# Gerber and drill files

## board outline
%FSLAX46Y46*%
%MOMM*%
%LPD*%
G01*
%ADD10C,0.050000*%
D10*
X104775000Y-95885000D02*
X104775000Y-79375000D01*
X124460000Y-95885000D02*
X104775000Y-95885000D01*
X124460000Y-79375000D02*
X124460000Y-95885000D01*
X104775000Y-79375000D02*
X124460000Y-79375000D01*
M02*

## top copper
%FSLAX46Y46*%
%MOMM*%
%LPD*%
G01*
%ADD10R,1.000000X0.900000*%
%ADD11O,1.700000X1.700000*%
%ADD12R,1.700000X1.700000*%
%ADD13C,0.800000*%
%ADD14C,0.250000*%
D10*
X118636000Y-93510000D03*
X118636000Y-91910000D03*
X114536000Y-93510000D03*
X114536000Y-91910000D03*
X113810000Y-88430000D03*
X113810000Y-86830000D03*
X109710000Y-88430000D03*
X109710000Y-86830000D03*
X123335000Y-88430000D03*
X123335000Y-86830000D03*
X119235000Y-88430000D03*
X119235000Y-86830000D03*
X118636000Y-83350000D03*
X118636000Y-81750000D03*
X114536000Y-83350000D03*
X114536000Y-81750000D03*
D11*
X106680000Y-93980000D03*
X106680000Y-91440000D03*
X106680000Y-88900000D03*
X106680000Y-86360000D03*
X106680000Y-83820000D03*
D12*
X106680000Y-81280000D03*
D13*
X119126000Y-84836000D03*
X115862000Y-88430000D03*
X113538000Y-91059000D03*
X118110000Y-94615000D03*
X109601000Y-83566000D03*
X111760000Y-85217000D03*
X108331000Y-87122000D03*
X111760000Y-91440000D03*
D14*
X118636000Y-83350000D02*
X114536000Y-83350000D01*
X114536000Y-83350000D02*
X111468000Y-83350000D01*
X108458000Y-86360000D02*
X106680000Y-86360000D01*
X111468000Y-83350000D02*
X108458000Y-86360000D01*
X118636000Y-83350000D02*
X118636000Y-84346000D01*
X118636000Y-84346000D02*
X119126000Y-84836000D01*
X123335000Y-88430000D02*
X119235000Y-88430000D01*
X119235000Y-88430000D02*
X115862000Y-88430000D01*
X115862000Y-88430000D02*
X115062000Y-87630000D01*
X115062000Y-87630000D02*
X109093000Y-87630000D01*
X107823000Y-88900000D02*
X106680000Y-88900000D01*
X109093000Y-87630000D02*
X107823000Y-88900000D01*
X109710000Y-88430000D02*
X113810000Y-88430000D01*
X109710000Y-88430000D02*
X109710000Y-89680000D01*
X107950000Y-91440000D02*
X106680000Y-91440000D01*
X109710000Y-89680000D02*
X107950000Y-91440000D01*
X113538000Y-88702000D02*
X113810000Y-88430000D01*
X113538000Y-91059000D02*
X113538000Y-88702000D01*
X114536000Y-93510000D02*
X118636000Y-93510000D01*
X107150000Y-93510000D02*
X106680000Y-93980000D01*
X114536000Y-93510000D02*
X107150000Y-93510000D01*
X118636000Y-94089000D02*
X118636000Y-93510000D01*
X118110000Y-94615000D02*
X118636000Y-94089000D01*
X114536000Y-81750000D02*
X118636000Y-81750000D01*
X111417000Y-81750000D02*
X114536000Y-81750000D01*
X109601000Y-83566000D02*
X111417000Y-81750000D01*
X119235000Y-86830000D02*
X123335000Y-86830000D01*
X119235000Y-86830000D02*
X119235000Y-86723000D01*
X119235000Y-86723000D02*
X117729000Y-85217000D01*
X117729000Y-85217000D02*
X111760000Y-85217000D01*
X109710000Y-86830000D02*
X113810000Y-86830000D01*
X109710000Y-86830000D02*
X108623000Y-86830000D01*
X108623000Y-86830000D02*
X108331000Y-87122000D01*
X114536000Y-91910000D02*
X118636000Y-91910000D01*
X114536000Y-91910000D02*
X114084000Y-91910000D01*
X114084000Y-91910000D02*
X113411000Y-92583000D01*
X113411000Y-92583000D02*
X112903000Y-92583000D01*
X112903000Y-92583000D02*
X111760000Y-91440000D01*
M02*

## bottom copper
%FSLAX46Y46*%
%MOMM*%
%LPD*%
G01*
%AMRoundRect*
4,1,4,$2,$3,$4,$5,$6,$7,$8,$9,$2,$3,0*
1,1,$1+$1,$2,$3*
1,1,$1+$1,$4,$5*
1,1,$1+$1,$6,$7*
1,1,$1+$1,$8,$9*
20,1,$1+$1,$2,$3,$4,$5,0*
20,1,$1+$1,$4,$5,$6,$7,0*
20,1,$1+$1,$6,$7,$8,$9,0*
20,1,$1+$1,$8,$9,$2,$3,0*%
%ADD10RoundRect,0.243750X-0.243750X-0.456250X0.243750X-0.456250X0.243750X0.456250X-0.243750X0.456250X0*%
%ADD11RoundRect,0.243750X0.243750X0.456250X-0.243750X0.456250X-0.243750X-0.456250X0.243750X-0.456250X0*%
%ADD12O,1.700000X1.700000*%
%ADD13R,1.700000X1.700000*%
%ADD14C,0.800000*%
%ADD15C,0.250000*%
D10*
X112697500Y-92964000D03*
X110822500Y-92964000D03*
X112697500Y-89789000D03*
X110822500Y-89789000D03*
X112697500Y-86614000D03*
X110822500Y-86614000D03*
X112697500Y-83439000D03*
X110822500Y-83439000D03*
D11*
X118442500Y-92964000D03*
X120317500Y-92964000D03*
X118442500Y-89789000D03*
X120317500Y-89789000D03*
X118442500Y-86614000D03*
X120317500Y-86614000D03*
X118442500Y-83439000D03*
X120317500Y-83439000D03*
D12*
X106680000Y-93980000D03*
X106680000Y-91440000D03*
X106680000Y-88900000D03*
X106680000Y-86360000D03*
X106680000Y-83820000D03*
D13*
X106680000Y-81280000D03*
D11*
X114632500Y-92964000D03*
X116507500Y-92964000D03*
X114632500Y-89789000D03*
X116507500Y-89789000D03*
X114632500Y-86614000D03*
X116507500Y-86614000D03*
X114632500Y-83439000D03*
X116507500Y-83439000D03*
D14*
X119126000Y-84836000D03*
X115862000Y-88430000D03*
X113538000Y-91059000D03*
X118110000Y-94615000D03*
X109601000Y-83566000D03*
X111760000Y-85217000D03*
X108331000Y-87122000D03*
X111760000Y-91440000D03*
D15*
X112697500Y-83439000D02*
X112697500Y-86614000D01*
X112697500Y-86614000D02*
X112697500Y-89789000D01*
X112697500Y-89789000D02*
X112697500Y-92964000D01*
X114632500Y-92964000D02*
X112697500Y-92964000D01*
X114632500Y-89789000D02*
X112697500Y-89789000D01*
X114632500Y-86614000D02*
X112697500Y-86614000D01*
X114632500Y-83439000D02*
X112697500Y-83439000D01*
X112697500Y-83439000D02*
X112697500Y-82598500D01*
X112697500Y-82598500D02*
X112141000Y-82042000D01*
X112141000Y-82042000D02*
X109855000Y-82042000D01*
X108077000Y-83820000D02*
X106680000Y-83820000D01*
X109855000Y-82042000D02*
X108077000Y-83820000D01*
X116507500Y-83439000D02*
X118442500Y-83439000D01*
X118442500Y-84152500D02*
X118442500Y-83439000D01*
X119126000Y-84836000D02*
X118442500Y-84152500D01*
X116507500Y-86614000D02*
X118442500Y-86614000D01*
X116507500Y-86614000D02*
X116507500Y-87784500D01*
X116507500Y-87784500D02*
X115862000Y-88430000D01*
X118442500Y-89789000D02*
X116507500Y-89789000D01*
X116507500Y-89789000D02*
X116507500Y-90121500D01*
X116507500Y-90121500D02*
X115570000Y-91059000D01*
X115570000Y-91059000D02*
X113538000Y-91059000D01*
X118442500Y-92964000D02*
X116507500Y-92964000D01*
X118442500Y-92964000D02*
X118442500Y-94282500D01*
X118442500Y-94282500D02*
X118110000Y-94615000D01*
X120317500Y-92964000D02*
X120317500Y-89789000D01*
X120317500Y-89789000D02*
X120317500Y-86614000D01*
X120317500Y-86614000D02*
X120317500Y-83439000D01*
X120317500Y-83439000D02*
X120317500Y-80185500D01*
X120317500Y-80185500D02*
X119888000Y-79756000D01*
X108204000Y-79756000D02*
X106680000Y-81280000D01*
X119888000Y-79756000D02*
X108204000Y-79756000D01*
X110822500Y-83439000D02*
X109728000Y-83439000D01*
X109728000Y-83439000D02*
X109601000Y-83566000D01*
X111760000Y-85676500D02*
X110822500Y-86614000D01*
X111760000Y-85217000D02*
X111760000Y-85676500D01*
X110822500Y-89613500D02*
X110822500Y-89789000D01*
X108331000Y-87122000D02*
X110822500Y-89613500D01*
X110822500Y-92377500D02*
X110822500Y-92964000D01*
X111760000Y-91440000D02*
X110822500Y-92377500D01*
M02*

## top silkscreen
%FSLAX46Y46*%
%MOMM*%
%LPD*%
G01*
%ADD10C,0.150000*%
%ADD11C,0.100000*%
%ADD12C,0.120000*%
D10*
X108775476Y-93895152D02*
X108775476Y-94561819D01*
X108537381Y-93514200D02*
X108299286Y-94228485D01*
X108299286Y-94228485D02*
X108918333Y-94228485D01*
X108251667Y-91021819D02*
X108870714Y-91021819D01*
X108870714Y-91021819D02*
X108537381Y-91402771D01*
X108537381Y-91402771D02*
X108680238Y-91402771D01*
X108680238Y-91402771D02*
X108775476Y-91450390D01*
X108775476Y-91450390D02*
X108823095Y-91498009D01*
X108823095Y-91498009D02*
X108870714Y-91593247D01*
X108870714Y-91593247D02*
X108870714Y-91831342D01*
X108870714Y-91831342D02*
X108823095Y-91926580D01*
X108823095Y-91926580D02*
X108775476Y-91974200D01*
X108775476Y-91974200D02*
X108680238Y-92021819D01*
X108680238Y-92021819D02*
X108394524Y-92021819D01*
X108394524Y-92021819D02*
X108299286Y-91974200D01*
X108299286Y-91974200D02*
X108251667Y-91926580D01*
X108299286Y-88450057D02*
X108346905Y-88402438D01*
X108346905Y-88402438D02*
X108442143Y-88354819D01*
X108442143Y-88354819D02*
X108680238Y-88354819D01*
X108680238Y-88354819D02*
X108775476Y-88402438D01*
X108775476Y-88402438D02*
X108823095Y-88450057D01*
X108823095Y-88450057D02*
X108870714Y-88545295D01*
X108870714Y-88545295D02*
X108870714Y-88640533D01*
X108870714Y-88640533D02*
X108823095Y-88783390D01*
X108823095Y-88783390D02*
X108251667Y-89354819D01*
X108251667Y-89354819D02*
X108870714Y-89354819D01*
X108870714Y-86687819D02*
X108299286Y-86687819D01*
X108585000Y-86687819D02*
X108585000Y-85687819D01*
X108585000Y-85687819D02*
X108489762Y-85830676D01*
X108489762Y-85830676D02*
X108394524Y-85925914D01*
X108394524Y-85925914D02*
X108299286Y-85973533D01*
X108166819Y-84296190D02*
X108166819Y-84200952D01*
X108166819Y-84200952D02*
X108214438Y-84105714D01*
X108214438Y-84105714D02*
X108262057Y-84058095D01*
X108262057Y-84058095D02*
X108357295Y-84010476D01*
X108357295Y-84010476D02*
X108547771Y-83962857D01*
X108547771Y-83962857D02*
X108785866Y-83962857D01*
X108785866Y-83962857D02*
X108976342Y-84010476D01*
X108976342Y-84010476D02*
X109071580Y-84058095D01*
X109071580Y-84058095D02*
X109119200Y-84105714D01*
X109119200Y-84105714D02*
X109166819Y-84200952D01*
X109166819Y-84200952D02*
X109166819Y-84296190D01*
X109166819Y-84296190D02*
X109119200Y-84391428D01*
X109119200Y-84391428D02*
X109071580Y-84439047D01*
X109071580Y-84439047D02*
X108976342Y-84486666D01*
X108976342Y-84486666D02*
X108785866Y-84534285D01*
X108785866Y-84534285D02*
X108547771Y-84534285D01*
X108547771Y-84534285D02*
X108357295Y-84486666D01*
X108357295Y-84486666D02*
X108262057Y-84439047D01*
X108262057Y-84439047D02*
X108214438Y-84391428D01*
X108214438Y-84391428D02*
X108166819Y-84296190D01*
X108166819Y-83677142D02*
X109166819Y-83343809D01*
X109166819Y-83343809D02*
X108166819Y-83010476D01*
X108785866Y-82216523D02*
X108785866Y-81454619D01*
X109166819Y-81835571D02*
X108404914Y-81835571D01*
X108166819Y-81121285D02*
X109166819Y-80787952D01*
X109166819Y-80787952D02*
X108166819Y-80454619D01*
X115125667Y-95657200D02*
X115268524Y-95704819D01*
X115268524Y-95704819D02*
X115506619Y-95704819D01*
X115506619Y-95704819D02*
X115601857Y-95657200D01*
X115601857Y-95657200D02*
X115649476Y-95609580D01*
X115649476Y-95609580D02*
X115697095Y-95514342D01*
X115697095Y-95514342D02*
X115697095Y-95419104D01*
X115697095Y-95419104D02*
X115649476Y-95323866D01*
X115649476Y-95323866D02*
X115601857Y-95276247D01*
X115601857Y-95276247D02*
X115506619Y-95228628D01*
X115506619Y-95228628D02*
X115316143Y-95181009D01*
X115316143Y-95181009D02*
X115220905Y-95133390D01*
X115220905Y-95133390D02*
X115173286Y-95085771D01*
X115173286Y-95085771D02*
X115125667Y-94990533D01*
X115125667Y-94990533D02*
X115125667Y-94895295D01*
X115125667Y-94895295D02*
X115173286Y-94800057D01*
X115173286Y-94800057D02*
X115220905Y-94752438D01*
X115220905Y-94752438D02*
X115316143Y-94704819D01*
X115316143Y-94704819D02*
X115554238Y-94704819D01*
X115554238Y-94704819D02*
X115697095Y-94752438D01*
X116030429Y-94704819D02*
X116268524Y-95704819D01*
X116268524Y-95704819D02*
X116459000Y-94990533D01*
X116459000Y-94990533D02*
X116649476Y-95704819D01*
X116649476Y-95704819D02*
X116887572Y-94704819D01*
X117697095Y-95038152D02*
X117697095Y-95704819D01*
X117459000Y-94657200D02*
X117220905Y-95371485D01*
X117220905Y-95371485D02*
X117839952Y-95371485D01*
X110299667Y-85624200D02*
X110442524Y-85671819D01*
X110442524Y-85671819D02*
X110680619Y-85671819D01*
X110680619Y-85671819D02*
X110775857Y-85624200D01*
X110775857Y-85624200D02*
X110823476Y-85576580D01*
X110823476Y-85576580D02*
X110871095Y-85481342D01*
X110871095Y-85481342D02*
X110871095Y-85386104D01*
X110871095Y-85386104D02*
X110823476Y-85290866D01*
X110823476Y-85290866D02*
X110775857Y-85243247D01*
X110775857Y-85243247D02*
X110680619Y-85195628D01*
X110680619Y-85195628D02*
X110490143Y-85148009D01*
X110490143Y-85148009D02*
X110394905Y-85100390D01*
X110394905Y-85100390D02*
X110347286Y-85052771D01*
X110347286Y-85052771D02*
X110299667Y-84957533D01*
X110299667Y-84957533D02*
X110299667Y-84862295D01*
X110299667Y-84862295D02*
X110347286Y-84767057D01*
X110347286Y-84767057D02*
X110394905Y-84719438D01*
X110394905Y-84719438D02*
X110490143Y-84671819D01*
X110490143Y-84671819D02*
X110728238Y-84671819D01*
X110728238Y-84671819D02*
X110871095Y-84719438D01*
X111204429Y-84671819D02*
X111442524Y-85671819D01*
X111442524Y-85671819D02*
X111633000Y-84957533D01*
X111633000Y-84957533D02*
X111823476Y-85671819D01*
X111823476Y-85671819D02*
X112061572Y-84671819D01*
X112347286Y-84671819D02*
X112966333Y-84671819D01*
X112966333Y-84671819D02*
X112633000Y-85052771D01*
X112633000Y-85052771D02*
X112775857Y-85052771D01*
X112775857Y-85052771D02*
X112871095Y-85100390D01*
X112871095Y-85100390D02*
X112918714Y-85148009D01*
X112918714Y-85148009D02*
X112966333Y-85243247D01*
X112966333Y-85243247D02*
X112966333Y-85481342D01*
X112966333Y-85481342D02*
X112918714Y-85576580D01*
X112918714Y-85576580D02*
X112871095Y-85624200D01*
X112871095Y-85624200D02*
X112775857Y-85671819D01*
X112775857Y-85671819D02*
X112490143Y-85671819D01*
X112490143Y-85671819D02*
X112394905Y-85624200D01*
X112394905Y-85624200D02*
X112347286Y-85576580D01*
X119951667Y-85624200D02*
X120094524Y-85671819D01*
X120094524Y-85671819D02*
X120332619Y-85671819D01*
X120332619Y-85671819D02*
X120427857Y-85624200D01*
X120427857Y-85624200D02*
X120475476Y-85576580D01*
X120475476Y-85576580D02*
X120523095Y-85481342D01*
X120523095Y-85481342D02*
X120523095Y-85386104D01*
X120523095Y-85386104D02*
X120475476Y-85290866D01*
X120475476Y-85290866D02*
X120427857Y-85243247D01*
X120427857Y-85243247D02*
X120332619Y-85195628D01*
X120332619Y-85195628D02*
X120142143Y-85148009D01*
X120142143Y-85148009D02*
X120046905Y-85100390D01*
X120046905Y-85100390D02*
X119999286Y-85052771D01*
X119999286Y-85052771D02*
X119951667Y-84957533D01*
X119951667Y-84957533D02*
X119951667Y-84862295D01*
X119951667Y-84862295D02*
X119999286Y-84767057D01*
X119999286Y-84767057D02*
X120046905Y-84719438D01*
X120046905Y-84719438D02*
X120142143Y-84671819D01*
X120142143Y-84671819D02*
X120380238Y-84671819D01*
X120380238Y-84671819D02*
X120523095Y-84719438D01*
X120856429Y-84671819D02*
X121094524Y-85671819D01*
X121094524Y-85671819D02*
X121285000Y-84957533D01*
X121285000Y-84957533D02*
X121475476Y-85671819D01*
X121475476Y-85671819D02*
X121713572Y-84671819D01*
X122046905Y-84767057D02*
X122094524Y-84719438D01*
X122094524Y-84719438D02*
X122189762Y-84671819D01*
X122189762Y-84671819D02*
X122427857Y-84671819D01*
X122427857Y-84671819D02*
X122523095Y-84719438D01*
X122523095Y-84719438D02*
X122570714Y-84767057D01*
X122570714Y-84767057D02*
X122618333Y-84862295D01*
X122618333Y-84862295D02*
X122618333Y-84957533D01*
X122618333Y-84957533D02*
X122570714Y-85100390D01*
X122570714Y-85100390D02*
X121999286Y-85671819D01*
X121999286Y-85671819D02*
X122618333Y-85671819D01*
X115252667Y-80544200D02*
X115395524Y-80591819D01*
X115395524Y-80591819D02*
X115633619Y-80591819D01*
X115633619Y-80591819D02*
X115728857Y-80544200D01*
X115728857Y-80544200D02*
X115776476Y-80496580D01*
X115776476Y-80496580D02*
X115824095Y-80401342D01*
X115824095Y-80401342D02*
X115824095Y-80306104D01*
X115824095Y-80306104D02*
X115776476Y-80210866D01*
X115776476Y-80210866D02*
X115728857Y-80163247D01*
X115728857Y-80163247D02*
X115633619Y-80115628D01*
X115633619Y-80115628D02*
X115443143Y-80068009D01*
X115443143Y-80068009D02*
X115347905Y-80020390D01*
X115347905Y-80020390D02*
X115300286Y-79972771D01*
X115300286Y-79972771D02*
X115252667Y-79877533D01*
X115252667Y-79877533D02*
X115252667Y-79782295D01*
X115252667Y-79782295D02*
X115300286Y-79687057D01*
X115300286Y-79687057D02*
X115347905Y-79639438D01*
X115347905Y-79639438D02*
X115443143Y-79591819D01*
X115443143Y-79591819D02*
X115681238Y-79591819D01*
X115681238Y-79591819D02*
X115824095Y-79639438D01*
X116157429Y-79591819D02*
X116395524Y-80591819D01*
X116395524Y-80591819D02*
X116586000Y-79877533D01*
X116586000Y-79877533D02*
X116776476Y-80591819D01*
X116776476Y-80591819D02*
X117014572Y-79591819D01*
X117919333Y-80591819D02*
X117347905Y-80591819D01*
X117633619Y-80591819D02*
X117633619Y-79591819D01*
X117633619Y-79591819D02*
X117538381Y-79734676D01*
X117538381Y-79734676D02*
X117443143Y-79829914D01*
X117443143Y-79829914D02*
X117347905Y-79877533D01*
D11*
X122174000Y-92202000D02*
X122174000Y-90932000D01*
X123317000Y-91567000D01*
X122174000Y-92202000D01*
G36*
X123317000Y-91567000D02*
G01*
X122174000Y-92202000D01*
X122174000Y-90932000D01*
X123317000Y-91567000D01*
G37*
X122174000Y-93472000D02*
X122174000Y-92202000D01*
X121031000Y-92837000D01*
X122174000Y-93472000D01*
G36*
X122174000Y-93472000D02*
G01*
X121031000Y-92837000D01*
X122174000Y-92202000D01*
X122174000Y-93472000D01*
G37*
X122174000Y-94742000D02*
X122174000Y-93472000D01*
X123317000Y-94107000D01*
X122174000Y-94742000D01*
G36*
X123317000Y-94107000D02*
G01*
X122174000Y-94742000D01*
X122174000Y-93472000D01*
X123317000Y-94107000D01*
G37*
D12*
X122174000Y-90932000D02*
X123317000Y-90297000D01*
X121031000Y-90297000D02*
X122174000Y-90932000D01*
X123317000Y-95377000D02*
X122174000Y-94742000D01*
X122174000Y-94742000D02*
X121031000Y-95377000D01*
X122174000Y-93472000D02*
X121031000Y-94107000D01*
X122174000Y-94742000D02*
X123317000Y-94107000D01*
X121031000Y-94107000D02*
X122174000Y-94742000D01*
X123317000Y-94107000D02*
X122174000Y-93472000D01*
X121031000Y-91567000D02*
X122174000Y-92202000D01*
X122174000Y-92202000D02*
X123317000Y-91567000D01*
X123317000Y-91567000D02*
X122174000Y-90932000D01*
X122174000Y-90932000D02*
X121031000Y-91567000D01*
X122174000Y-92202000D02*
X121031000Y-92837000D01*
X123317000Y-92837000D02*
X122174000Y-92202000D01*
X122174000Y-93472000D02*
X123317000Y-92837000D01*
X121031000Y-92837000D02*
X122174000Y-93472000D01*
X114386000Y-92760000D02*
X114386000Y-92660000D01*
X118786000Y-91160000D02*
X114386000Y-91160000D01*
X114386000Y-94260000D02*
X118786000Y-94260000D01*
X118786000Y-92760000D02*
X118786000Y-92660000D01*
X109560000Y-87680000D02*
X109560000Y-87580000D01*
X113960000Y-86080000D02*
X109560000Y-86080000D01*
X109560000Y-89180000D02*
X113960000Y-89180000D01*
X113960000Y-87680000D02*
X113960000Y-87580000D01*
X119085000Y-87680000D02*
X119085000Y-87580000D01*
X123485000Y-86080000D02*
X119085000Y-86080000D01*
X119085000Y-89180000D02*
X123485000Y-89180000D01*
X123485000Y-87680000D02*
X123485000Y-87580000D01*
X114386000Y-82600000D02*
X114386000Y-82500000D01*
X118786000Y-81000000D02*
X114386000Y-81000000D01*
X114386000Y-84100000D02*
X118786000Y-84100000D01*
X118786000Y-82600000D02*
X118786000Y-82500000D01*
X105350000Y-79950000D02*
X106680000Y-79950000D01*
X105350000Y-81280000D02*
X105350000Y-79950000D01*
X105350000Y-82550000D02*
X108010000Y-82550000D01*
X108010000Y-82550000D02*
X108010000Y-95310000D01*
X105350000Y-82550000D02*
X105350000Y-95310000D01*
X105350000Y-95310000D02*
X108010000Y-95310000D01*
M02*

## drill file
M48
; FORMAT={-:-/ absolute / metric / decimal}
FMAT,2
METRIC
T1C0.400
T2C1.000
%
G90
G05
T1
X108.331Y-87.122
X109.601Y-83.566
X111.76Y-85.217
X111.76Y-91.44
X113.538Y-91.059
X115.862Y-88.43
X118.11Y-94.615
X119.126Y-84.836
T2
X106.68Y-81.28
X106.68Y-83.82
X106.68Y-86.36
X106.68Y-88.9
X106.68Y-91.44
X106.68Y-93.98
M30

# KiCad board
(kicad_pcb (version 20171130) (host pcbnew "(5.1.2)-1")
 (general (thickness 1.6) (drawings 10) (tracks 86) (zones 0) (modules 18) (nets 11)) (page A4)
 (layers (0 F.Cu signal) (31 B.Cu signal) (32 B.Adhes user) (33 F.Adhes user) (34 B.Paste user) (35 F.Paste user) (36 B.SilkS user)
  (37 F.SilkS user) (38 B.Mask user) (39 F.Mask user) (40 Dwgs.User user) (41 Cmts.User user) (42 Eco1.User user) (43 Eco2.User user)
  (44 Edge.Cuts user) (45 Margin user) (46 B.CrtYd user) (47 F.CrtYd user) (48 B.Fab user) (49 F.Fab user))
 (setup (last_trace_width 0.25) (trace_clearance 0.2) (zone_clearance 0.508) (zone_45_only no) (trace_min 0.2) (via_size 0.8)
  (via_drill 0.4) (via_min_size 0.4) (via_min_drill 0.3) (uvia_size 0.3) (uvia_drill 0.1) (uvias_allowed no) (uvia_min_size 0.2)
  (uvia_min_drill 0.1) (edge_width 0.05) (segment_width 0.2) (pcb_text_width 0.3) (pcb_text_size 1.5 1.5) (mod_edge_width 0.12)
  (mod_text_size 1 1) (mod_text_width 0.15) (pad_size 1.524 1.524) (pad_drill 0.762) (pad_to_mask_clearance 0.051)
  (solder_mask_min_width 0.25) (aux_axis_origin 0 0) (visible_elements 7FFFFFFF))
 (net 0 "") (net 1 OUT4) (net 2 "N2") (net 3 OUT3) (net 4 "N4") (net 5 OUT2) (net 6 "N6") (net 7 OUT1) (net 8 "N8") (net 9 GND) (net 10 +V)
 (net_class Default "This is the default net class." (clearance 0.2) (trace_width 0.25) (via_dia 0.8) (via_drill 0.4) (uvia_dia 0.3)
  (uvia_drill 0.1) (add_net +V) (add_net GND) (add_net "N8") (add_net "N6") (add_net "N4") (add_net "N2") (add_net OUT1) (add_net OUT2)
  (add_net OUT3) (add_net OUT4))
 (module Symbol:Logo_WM (layer F.Cu) (at 122.174 92.837 90)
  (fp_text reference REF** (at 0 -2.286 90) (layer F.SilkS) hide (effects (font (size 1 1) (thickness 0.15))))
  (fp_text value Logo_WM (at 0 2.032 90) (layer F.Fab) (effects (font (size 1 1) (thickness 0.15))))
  (fp_poly (pts (xy 0.635 0) (xy 1.905 0) (xy 1.27 1.143)) (layer F.SilkS) (width 0.1))
  (fp_poly (pts (xy -0.635 0) (xy 0.635 0) (xy 0 -1.143)) (layer F.SilkS) (width 0.1))
  (fp_poly (pts (xy -1.905 0) (xy -0.635 0) (xy -1.27 1.143)) (layer F.SilkS) (width 0.1))
  (fp_line (start 1.905 0) (end 2.54 1.143) (layer F.SilkS) (width 0.12))
  (fp_line (start 2.54 -1.143) (end 1.905 0) (layer F.SilkS) (width 0.12))
  (fp_line (start -2.54 1.143) (end -1.905 0) (layer F.SilkS) (width 0.12))
  (fp_line (start -1.905 0) (end -2.54 -1.143) (layer F.SilkS) (width 0.12))
  (fp_line (start -0.635 0) (end -1.27 -1.143) (layer F.SilkS) (width 0.12))
  (fp_line (start -1.905 0) (end -1.27 1.143) (layer F.SilkS) (width 0.12))
  (fp_line (start -1.27 -1.143) (end -1.905 0) (layer F.SilkS) (width 0.12))
  (fp_line (start -1.27 1.143) (end -0.635 0) (layer F.SilkS) (width 0.12))
  (fp_line (start 1.27 -1.143) (end 0.635 0) (layer F.SilkS) (width 0.12))
  (fp_line (start 0.635 0) (end 1.27 1.143) (layer F.SilkS) (width 0.12))
  (fp_line (start 1.27 1.143) (end 1.905 0) (layer F.SilkS) (width 0.12))
  (fp_line (start 1.905 0) (end 1.27 -1.143) (layer F.SilkS) (width 0.12))
  (fp_line (start 0.635 0) (end 0 -1.143) (layer F.SilkS) (width 0.12))
  (fp_line (start 0 1.143) (end 0.635 0) (layer F.SilkS) (width 0.12))
  (fp_line (start -0.635 0) (end 0 1.143) (layer F.SilkS) (width 0.12))
  (fp_line (start 0 -1.143) (end -0.635 0) (layer F.SilkS) (width 0.12)))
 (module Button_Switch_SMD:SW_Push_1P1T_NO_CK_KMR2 (layer F.Cu) (at 116.586 92.71)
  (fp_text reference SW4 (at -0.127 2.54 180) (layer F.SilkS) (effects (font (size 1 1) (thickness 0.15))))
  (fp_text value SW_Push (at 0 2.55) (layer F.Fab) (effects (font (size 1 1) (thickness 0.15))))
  (fp_line (start -2.2 0.05) (end -2.2 -0.05) (layer F.SilkS) (width 0.12))
  (fp_line (start 2.2 -1.55) (end -2.2 -1.55) (layer F.SilkS) (width 0.12))
  (fp_line (start -2.2 1.55) (end 2.2 1.55) (layer F.SilkS) (width 0.12))
  (fp_line (start 2.2 0.05) (end 2.2 -0.05) (layer F.SilkS) (width 0.12))
  (pad 2 smd rect (at 2.05 0.8 90) (size 0.9 1) (layers F.Cu F.Paste F.Mask) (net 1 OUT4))
  (pad 1 smd rect (at 2.05 -0.8 90) (size 0.9 1) (layers F.Cu F.Paste F.Mask) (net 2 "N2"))
  (pad 2 smd rect (at -2.05 0.8 90) (size 0.9 1) (layers F.Cu F.Paste F.Mask) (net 1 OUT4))
  (pad 1 smd rect (at -2.05 -0.8 90) (size 0.9 1) (layers F.Cu F.Paste F.Mask) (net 2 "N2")))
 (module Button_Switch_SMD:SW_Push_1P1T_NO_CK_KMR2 (layer F.Cu) (at 111.76 87.63)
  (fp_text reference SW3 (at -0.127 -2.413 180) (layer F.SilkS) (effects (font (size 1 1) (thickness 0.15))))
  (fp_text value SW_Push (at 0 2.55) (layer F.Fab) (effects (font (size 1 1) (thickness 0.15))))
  (fp_line (start -2.2 0.05) (end -2.2 -0.05) (layer F.SilkS) (width 0.12))
  (fp_line (start 2.2 -1.55) (end -2.2 -1.55) (layer F.SilkS) (width 0.12))
  (fp_line (start -2.2 1.55) (end 2.2 1.55) (layer F.SilkS) (width 0.12))
  (fp_line (start 2.2 0.05) (end 2.2 -0.05) (layer F.SilkS) (width 0.12))
  (pad 2 smd rect (at 2.05 0.8 90) (size 0.9 1) (layers F.Cu F.Paste F.Mask) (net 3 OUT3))
  (pad 1 smd rect (at 2.05 -0.8 90) (size 0.9 1) (layers F.Cu F.Paste F.Mask) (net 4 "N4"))
  (pad 2 smd rect (at -2.05 0.8 90) (size 0.9 1) (layers F.Cu F.Paste F.Mask) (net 3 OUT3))
  (pad 1 smd rect (at -2.05 -0.8 90) (size 0.9 1) (layers F.Cu F.Paste F.Mask) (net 4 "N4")))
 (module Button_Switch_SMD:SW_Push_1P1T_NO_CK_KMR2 (layer F.Cu) (at 121.285 87.63)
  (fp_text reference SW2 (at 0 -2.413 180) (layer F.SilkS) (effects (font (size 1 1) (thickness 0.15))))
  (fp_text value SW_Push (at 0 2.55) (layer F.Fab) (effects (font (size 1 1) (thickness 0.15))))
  (fp_line (start -2.2 0.05) (end -2.2 -0.05) (layer F.SilkS) (width 0.12))
  (fp_line (start 2.2 -1.55) (end -2.2 -1.55) (layer F.SilkS) (width 0.12))
  (fp_line (start -2.2 1.55) (end 2.2 1.55) (layer F.SilkS) (width 0.12))
  (fp_line (start 2.2 0.05) (end 2.2 -0.05) (layer F.SilkS) (width 0.12))
  (pad 2 smd rect (at 2.05 0.8 90) (size 0.9 1) (layers F.Cu F.Paste F.Mask) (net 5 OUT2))
  (pad 1 smd rect (at 2.05 -0.8 90) (size 0.9 1) (layers F.Cu F.Paste F.Mask) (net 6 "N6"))
  (pad 2 smd rect (at -2.05 0.8 90) (size 0.9 1) (layers F.Cu F.Paste F.Mask) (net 5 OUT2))
  (pad 1 smd rect (at -2.05 -0.8 90) (size 0.9 1) (layers F.Cu F.Paste F.Mask) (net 6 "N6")))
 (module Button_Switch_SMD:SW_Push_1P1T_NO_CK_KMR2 (layer F.Cu) (at 116.586 82.55)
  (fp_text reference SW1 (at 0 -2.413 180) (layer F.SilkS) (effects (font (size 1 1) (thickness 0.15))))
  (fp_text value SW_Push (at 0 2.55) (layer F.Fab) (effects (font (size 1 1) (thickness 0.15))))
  (fp_line (start -2.2 0.05) (end -2.2 -0.05) (layer F.SilkS) (width 0.12))
  (fp_line (start 2.2 -1.55) (end -2.2 -1.55) (layer F.SilkS) (width 0.12))
  (fp_line (start -2.2 1.55) (end 2.2 1.55) (layer F.SilkS) (width 0.12))
  (fp_line (start 2.2 0.05) (end 2.2 -0.05) (layer F.SilkS) (width 0.12))
  (pad 2 smd rect (at 2.05 0.8 90) (size 0.9 1) (layers F.Cu F.Paste F.Mask) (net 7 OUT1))
  (pad 1 smd rect (at 2.05 -0.8 90) (size 0.9 1) (layers F.Cu F.Paste F.Mask) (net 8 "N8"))
  (pad 2 smd rect (at -2.05 0.8 90) (size 0.9 1) (layers F.Cu F.Paste F.Mask) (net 7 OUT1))
  (pad 1 smd rect (at -2.05 -0.8 90) (size 0.9 1) (layers F.Cu F.Paste F.Mask) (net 8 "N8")))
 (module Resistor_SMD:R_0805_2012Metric (layer B.Cu) (at 111.76 92.964)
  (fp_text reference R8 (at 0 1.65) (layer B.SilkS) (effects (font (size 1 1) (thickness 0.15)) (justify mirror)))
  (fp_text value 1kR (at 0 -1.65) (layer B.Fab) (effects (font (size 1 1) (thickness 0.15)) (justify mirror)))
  (pad 2 smd roundrect (at 0.9375 0) (size 0.975 1.4) (layers B.Cu B.Paste B.Mask) (roundrect_rratio 0.25) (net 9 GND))
  (pad 1 smd roundrect (at -0.9375 0) (size 0.975 1.4) (layers B.Cu B.Paste B.Mask) (roundrect_rratio 0.25) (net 2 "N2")))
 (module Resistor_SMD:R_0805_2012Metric (layer B.Cu) (at 111.76 89.789)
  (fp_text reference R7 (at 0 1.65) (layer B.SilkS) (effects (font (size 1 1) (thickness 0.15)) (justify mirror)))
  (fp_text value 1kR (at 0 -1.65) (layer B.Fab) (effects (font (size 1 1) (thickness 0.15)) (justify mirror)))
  (pad 2 smd roundrect (at 0.9375 0) (size 0.975 1.4) (layers B.Cu B.Paste B.Mask) (roundrect_rratio 0.25) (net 9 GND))
  (pad 1 smd roundrect (at -0.9375 0) (size 0.975 1.4) (layers B.Cu B.Paste B.Mask) (roundrect_rratio 0.25) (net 4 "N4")))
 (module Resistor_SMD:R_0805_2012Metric (layer B.Cu) (at 111.76 86.614)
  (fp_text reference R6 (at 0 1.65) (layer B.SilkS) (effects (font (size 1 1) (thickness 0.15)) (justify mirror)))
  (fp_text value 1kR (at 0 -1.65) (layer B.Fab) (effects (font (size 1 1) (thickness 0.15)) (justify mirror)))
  (pad 2 smd roundrect (at 0.9375 0) (size 0.975 1.4) (layers B.Cu B.Paste B.Mask) (roundrect_rratio 0.25) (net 9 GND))
  (pad 1 smd roundrect (at -0.9375 0) (size 0.975 1.4) (layers B.Cu B.Paste B.Mask) (roundrect_rratio 0.25) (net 6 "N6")))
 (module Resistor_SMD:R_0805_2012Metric (layer B.Cu) (at 111.76 83.439)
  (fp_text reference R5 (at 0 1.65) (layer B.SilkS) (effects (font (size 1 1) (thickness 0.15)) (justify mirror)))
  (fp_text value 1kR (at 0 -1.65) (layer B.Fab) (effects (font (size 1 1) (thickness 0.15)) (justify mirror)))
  (pad 2 smd roundrect (at 0.9375 0) (size 0.975 1.4) (layers B.Cu B.Paste B.Mask) (roundrect_rratio 0.25) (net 9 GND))
  (pad 1 smd roundrect (at -0.9375 0) (size 0.975 1.4) (layers B.Cu B.Paste B.Mask) (roundrect_rratio 0.25) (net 8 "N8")))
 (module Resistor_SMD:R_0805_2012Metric (layer B.Cu) (at 119.38 92.964 180)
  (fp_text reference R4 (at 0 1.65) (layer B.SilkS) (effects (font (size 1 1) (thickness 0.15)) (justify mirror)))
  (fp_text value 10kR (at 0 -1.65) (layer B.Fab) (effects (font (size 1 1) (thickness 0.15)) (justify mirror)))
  (pad 2 smd roundrect (at 0.9375 0 180) (size 0.975 1.4) (layers B.Cu B.Paste B.Mask) (roundrect_rratio 0.25) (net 1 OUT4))
  (pad 1 smd roundrect (at -0.9375 0 180) (size 0.975 1.4) (layers B.Cu B.Paste B.Mask) (roundrect_rratio 0.25) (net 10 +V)))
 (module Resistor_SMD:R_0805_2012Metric (layer B.Cu) (at 119.38 89.789 180)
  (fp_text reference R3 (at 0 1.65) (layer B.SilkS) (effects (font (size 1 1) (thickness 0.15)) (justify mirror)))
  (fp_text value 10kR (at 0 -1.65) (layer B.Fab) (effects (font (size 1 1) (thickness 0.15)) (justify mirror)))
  (pad 2 smd roundrect (at 0.9375 0 180) (size 0.975 1.4) (layers B.Cu B.Paste B.Mask) (roundrect_rratio 0.25) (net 3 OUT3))
  (pad 1 smd roundrect (at -0.9375 0 180) (size 0.975 1.4) (layers B.Cu B.Paste B.Mask) (roundrect_rratio 0.25) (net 10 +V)))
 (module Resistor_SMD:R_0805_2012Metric (layer B.Cu) (at 119.38 86.614 180)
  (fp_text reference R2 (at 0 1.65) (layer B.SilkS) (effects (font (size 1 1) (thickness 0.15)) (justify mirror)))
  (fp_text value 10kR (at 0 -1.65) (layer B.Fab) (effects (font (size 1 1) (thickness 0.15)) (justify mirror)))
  (pad 2 smd roundrect (at 0.9375 0 180) (size 0.975 1.4) (layers B.Cu B.Paste B.Mask) (roundrect_rratio 0.25) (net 5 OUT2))
  (pad 1 smd roundrect (at -0.9375 0 180) (size 0.975 1.4) (layers B.Cu B.Paste B.Mask) (roundrect_rratio 0.25) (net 10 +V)))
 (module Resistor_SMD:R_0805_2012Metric (layer B.Cu) (at 119.38 83.439 180)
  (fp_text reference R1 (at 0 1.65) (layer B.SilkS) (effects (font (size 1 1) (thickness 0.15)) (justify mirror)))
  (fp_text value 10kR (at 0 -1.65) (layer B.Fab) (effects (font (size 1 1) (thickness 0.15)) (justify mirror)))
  (pad 2 smd roundrect (at 0.9375 0 180) (size 0.975 1.4) (layers B.Cu B.Paste B.Mask) (roundrect_rratio 0.25) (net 7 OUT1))
  (pad 1 smd roundrect (at -0.9375 0 180) (size 0.975 1.4) (layers B.Cu B.Paste B.Mask) (roundrect_rratio 0.25) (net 10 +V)))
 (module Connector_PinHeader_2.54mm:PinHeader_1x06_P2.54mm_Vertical (layer F.Cu) (at 106.68 81.28)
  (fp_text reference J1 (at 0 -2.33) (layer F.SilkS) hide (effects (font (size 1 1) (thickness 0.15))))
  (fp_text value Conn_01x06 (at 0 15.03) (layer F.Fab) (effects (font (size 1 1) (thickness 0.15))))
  (fp_line (start -1.33 -1.33) (end 0 -1.33) (layer F.SilkS) (width 0.12))
  (fp_line (start -1.33 0) (end -1.33 -1.33) (layer F.SilkS) (width 0.12))
  (fp_line (start -1.33 1.27) (end 1.33 1.27) (layer F.SilkS) (width 0.12))
  (fp_line (start 1.33 1.27) (end 1.33 14.03) (layer F.SilkS) (width 0.12))
  (fp_line (start -1.33 1.27) (end -1.33 14.03) (layer F.SilkS) (width 0.12))
  (fp_line (start -1.33 14.03) (end 1.33 14.03) (layer F.SilkS) (width 0.12))
  (pad 6 thru_hole oval (at 0 12.7) (size 1.7 1.7) (drill 1) (layers *.Cu *.Mask) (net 1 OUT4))
  (pad 5 thru_hole oval (at 0 10.16) (size 1.7 1.7) (drill 1) (layers *.Cu *.Mask) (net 3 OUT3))
  (pad 4 thru_hole oval (at 0 7.62) (size 1.7 1.7) (drill 1) (layers *.Cu *.Mask) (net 5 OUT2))
  (pad 3 thru_hole oval (at 0 5.08) (size 1.7 1.7) (drill 1) (layers *.Cu *.Mask) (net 7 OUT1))
  (pad 2 thru_hole oval (at 0 2.54) (size 1.7 1.7) (drill 1) (layers *.Cu *.Mask) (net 9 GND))
  (pad 1 thru_hole rect (at 0 0) (size 1.7 1.7) (drill 1) (layers *.Cu *.Mask) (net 10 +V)))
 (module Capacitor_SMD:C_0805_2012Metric (layer B.Cu) (at 115.57 92.964 180)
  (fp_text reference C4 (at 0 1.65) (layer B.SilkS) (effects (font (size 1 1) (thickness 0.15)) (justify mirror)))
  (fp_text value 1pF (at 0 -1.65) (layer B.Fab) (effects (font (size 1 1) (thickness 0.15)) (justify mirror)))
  (pad 2 smd roundrect (at 0.9375 0 180) (size 0.975 1.4) (layers B.Cu B.Paste B.Mask) (roundrect_rratio 0.25) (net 9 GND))
  (pad 1 smd roundrect (at -0.9375 0 180) (size 0.975 1.4) (layers B.Cu B.Paste B.Mask) (roundrect_rratio 0.25) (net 1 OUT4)))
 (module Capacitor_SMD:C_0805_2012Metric (layer B.Cu) (at 115.57 89.789 180)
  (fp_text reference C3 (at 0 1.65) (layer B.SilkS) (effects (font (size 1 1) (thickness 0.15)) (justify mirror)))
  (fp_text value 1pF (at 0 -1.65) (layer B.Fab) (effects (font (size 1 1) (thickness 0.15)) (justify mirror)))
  (pad 2 smd roundrect (at 0.9375 0 180) (size 0.975 1.4) (layers B.Cu B.Paste B.Mask) (roundrect_rratio 0.25) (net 9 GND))
  (pad 1 smd roundrect (at -0.9375 0 180) (size 0.975 1.4) (layers B.Cu B.Paste B.Mask) (roundrect_rratio 0.25) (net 3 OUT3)))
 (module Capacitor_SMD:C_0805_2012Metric (layer B.Cu) (at 115.57 86.614 180)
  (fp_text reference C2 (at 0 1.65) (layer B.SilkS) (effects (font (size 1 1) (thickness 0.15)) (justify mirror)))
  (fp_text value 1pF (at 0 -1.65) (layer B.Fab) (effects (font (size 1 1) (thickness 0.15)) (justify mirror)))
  (pad 2 smd roundrect (at 0.9375 0 180) (size 0.975 1.4) (layers B.Cu B.Paste B.Mask) (roundrect_rratio 0.25) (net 9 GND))
  (pad 1 smd roundrect (at -0.9375 0 180) (size 0.975 1.4) (layers B.Cu B.Paste B.Mask) (roundrect_rratio 0.25) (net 5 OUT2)))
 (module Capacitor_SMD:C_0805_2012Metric (layer B.Cu) (at 115.57 83.439 180)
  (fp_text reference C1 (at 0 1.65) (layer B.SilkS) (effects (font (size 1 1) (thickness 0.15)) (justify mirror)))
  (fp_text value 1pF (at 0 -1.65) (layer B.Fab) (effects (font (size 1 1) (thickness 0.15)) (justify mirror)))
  (pad 2 smd roundrect (at 0.9375 0 180) (size 0.975 1.4) (layers B.Cu B.Paste B.Mask) (roundrect_rratio 0.25) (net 9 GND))
  (pad 1 smd roundrect (at -0.9375 0 180) (size 0.975 1.4) (layers B.Cu B.Paste B.Mask) (roundrect_rratio 0.25) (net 7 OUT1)))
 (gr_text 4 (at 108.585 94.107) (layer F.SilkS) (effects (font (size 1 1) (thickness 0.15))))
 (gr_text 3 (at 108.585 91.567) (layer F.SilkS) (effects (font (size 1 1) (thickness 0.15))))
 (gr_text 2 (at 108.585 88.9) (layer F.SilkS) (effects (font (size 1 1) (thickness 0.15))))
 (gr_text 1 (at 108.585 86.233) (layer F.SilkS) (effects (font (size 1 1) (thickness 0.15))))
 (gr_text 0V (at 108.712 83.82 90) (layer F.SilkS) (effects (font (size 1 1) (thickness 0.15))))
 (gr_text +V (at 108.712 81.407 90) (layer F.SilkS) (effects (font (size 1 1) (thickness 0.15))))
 (gr_line (start 104.775 95.885) (end 104.775 79.375) (layer Edge.Cuts) (width 0.05))
 (gr_line (start 124.46 95.885) (end 104.775 95.885) (layer Edge.Cuts) (width 0.05))
 (gr_line (start 124.46 79.375) (end 124.46 95.885) (layer Edge.Cuts) (width 0.05))
 (gr_line (start 104.775 79.375) (end 124.46 79.375) (layer Edge.Cuts) (width 0.05))
 (segment (start 112.6975 83.439) (end 112.6975 86.614) (width 0.25) (layer B.Cu) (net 9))
 (segment (start 112.6975 86.614) (end 112.6975 89.789) (width 0.25) (layer B.Cu) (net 9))
 (segment (start 112.6975 89.789) (end 112.6975 92.964) (width 0.25) (layer B.Cu) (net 9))
 (segment (start 114.6325 92.964) (end 112.6975 92.964) (width 0.25) (layer B.Cu) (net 9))
 (segment (start 114.6325 89.789) (end 112.6975 89.789) (width 0.25) (layer B.Cu) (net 9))
 (segment (start 114.6325 86.614) (end 112.6975 86.614) (width 0.25) (layer B.Cu) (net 9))
 (segment (start 114.6325 83.439) (end 112.6975 83.439) (width 0.25) (layer B.Cu) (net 9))
 (segment (start 112.6975 83.439) (end 112.6975 82.5985) (width 0.25) (layer B.Cu) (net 9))
 (segment (start 112.6975 82.5985) (end 112.141 82.042) (width 0.25) (layer B.Cu) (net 9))
 (segment (start 112.141 82.042) (end 109.855 82.042) (width 0.25) (layer B.Cu) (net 9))
 (segment (start 108.077 83.82) (end 106.68 83.82) (width 0.25) (layer B.Cu) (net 9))
 (segment (start 109.855 82.042) (end 108.077 83.82) (width 0.25) (layer B.Cu) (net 9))
 (segment (start 118.636 83.35) (end 114.536 83.35) (width 0.25) (layer F.Cu) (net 7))
 (segment (start 114.536 83.35) (end 111.468 83.35) (width 0.25) (layer F.Cu) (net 7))
 (segment (start 108.458 86.36) (end 106.68 86.36) (width 0.25) (layer F.Cu) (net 7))
 (segment (start 111.468 83.35) (end 108.458 86.36) (width 0.25) (layer F.Cu) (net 7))
 (segment (start 116.5075 83.439) (end 118.4425 83.439) (width 0.25) (layer B.Cu) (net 7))
 (via (at 119.126 84.836) (size 0.8) (drill 0.4) (layers F.Cu B.Cu) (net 7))
 (segment (start 118.636 83.35) (end 118.636 84.346) (width 0.25) (layer F.Cu) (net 7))
 (segment (start 118.636 84.346) (end 119.126 84.836) (width 0.25) (layer F.Cu) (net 7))
 (segment (start 118.4425 84.1525) (end 118.4425 83.439) (width 0.25) (layer B.Cu) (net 7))
 (segment (start 119.126 84.836) (end 118.4425 84.1525) (width 0.25) (layer B.Cu) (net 7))
 (segment (start 123.335 88.43) (end 119.235 88.43) (width 0.25) (layer F.Cu) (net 5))
 (segment (start 119.235 88.43) (end 115.862 88.43) (width 0.25) (layer F.Cu) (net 5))
 (segment (start 115.862 88.43) (end 115.062 87.63) (width 0.25) (layer F.Cu) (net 5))
 (segment (start 115.062 87.63) (end 109.093 87.63) (width 0.25) (layer F.Cu) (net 5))
 (segment (start 107.823 88.9) (end 106.68 88.9) (width 0.25) (layer F.Cu) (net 5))
 (segment (start 109.093 87.63) (end 107.823 88.9) (width 0.25) (layer F.Cu) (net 5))
 (segment (start 116.5075 86.614) (end 118.4425 86.614) (width 0.25) (layer B.Cu) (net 5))
 (via (at 115.862 88.43) (size 0.8) (drill 0.4) (layers F.Cu B.Cu) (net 5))
 (segment (start 116.5075 86.614) (end 116.5075 87.7845) (width 0.25) (layer B.Cu) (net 5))
 (segment (start 116.5075 87.7845) (end 115.862 88.43) (width 0.25) (layer B.Cu) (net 5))
 (segment (start 109.71 88.43) (end 113.81 88.43) (width 0.25) (layer F.Cu) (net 3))
 (segment (start 109.71 88.43) (end 109.71 89.68) (width 0.25) (layer F.Cu) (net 3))
 (segment (start 107.95 91.44) (end 106.68 91.44) (width 0.25) (layer F.Cu) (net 3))
 (segment (start 109.71 89.68) (end 107.95 91.44) (width 0.25) (layer F.Cu) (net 3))
 (segment (start 118.4425 89.789) (end 116.5075 89.789) (width 0.25) (layer B.Cu) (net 3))
 (segment (start 116.5075 89.789) (end 116.5075 90.1215) (width 0.25) (layer B.Cu) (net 3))
 (via (at 113.538 91.059) (size 0.8) (drill 0.4) (layers F.Cu B.Cu) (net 3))
 (segment (start 116.5075 90.1215) (end 115.57 91.059) (width 0.25) (layer B.Cu) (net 3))
 (segment (start 115.57 91.059) (end 113.538 91.059) (width 0.25) (layer B.Cu) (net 3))
 (segment (start 113.538 88.702) (end 113.81 88.43) (width 0.25) (layer F.Cu) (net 3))
 (segment (start 113.538 91.059) (end 113.538 88.702) (width 0.25) (layer F.Cu) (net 3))
 (segment (start 114.536 93.51) (end 118.636 93.51) (width 0.25) (layer F.Cu) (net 1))
 (segment (start 107.15 93.51) (end 106.68 93.98) (width 0.25) (layer F.Cu) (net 1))
 (segment (start 114.536 93.51) (end 107.15 93.51) (width 0.25) (layer F.Cu) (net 1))
 (segment (start 118.4425 92.964) (end 116.5075 92.964) (width 0.25) (layer B.Cu) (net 1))
 (via (at 118.11 94.615) (size 0.8) (drill 0.4) (layers F.Cu B.Cu) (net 1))
 (segment (start 118.4425 92.964) (end 118.4425 94.2825) (width 0.25) (layer B.Cu) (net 1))
 (segment (start 118.4425 94.2825) (end 118.11 94.615) (width 0.25) (layer B.Cu) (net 1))
 (segment (start 118.636 94.089) (end 118.636 93.51) (width 0.25) (layer F.Cu) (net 1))
 (segment (start 118.11 94.615) (end 118.636 94.089) (width 0.25) (layer F.Cu) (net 1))
 (segment (start 120.3175 92.964) (end 120.3175 89.789) (width 0.25) (layer B.Cu) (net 10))
 (segment (start 120.3175 89.789) (end 120.3175 86.614) (width 0.25) (layer B.Cu) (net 10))
 (segment (start 120.3175 86.614) (end 120.3175 83.439) (width 0.25) (layer B.Cu) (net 10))
 (segment (start 120.3175 83.439) (end 120.3175 80.1855) (width 0.25) (layer B.Cu) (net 10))
 (segment (start 120.3175 80.1855) (end 119.888 79.756) (width 0.25) (layer B.Cu) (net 10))
 (segment (start 108.204 79.756) (end 106.68 81.28) (width 0.25) (layer B.Cu) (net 10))
 (segment (start 119.888 79.756) (end 108.204 79.756) (width 0.25) (layer B.Cu) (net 10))
 (segment (start 114.536 81.75) (end 118.636 81.75) (width 0.25) (layer F.Cu) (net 8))
 (via (at 109.601 83.566) (size 0.8) (drill 0.4) (layers F.Cu B.Cu) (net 8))
 (segment (start 110.8225 83.439) (end 109.728 83.439) (width 0.25) (layer B.Cu) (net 8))
 (segment (start 109.728 83.439) (end 109.601 83.566) (width 0.25) (layer B.Cu) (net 8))
 (segment (start 111.417 81.75) (end 114.536 81.75) (width 0.25) (layer F.Cu) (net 8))
 (segment (start 109.601 83.566) (end 111.417 81.75) (width 0.25) (layer F.Cu) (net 8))
 (segment (start 119.235 86.83) (end 123.335 86.83) (width 0.25) (layer F.Cu) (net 6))
 (segment (start 119.235 86.83) (end 119.235 86.723) (width 0.25) (layer F.Cu) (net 6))
 (via (at 111.76 85.217) (size 0.8) (drill 0.4) (layers F.Cu B.Cu) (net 6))
 (segment (start 119.235 86.723) (end 117.729 85.217) (width 0.25) (layer F.Cu) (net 6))
 (segment (start 117.729 85.217) (end 111.76 85.217) (width 0.25) (layer F.Cu) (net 6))
 (segment (start 111.76 85.6765) (end 110.8225 86.614) (width 0.25) (layer B.Cu) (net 6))
 (segment (start 111.76 85.217) (end 111.76 85.6765) (width 0.25) (layer B.Cu) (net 6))
 (segment (start 109.71 86.83) (end 113.81 86.83) (width 0.25) (layer F.Cu) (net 4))
 (via (at 108.331 87.122) (size 0.8) (drill 0.4) (layers F.Cu B.Cu) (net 4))
 (segment (start 109.71 86.83) (end 108.623 86.83) (width 0.25) (layer F.Cu) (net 4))
 (segment (start 108.623 86.83) (end 108.331 87.122) (width 0.25) (layer F.Cu) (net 4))
 (segment (start 110.8225 89.6135) (end 110.8225 89.789) (width 0.25) (layer B.Cu) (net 4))
 (segment (start 108.331 87.122) (end 110.8225 89.6135) (width 0.25) (layer B.Cu) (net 4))
 (segment (start 114.536 91.91) (end 118.636 91.91) (width 0.25) (layer F.Cu) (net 2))
 (segment (start 114.536 91.91) (end 114.084 91.91) (width 0.25) (layer F.Cu) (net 2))
 (segment (start 114.084 91.91) (end 113.411 92.583) (width 0.25) (layer F.Cu) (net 2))
 (via (at 111.76 91.44) (size 0.8) (drill 0.4) (layers F.Cu B.Cu) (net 2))
 (segment (start 113.411 92.583) (end 112.903 92.583) (width 0.25) (layer F.Cu) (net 2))
 (segment (start 112.903 92.583) (end 111.76 91.44) (width 0.25) (layer F.Cu) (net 2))
 (segment (start 110.8225 92.3775) (end 110.8225 92.964) (width 0.25) (layer B.Cu) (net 2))
 (segment (start 111.76 91.44) (end 110.8225 92.3775) (width 0.25) (layer B.Cu) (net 2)))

